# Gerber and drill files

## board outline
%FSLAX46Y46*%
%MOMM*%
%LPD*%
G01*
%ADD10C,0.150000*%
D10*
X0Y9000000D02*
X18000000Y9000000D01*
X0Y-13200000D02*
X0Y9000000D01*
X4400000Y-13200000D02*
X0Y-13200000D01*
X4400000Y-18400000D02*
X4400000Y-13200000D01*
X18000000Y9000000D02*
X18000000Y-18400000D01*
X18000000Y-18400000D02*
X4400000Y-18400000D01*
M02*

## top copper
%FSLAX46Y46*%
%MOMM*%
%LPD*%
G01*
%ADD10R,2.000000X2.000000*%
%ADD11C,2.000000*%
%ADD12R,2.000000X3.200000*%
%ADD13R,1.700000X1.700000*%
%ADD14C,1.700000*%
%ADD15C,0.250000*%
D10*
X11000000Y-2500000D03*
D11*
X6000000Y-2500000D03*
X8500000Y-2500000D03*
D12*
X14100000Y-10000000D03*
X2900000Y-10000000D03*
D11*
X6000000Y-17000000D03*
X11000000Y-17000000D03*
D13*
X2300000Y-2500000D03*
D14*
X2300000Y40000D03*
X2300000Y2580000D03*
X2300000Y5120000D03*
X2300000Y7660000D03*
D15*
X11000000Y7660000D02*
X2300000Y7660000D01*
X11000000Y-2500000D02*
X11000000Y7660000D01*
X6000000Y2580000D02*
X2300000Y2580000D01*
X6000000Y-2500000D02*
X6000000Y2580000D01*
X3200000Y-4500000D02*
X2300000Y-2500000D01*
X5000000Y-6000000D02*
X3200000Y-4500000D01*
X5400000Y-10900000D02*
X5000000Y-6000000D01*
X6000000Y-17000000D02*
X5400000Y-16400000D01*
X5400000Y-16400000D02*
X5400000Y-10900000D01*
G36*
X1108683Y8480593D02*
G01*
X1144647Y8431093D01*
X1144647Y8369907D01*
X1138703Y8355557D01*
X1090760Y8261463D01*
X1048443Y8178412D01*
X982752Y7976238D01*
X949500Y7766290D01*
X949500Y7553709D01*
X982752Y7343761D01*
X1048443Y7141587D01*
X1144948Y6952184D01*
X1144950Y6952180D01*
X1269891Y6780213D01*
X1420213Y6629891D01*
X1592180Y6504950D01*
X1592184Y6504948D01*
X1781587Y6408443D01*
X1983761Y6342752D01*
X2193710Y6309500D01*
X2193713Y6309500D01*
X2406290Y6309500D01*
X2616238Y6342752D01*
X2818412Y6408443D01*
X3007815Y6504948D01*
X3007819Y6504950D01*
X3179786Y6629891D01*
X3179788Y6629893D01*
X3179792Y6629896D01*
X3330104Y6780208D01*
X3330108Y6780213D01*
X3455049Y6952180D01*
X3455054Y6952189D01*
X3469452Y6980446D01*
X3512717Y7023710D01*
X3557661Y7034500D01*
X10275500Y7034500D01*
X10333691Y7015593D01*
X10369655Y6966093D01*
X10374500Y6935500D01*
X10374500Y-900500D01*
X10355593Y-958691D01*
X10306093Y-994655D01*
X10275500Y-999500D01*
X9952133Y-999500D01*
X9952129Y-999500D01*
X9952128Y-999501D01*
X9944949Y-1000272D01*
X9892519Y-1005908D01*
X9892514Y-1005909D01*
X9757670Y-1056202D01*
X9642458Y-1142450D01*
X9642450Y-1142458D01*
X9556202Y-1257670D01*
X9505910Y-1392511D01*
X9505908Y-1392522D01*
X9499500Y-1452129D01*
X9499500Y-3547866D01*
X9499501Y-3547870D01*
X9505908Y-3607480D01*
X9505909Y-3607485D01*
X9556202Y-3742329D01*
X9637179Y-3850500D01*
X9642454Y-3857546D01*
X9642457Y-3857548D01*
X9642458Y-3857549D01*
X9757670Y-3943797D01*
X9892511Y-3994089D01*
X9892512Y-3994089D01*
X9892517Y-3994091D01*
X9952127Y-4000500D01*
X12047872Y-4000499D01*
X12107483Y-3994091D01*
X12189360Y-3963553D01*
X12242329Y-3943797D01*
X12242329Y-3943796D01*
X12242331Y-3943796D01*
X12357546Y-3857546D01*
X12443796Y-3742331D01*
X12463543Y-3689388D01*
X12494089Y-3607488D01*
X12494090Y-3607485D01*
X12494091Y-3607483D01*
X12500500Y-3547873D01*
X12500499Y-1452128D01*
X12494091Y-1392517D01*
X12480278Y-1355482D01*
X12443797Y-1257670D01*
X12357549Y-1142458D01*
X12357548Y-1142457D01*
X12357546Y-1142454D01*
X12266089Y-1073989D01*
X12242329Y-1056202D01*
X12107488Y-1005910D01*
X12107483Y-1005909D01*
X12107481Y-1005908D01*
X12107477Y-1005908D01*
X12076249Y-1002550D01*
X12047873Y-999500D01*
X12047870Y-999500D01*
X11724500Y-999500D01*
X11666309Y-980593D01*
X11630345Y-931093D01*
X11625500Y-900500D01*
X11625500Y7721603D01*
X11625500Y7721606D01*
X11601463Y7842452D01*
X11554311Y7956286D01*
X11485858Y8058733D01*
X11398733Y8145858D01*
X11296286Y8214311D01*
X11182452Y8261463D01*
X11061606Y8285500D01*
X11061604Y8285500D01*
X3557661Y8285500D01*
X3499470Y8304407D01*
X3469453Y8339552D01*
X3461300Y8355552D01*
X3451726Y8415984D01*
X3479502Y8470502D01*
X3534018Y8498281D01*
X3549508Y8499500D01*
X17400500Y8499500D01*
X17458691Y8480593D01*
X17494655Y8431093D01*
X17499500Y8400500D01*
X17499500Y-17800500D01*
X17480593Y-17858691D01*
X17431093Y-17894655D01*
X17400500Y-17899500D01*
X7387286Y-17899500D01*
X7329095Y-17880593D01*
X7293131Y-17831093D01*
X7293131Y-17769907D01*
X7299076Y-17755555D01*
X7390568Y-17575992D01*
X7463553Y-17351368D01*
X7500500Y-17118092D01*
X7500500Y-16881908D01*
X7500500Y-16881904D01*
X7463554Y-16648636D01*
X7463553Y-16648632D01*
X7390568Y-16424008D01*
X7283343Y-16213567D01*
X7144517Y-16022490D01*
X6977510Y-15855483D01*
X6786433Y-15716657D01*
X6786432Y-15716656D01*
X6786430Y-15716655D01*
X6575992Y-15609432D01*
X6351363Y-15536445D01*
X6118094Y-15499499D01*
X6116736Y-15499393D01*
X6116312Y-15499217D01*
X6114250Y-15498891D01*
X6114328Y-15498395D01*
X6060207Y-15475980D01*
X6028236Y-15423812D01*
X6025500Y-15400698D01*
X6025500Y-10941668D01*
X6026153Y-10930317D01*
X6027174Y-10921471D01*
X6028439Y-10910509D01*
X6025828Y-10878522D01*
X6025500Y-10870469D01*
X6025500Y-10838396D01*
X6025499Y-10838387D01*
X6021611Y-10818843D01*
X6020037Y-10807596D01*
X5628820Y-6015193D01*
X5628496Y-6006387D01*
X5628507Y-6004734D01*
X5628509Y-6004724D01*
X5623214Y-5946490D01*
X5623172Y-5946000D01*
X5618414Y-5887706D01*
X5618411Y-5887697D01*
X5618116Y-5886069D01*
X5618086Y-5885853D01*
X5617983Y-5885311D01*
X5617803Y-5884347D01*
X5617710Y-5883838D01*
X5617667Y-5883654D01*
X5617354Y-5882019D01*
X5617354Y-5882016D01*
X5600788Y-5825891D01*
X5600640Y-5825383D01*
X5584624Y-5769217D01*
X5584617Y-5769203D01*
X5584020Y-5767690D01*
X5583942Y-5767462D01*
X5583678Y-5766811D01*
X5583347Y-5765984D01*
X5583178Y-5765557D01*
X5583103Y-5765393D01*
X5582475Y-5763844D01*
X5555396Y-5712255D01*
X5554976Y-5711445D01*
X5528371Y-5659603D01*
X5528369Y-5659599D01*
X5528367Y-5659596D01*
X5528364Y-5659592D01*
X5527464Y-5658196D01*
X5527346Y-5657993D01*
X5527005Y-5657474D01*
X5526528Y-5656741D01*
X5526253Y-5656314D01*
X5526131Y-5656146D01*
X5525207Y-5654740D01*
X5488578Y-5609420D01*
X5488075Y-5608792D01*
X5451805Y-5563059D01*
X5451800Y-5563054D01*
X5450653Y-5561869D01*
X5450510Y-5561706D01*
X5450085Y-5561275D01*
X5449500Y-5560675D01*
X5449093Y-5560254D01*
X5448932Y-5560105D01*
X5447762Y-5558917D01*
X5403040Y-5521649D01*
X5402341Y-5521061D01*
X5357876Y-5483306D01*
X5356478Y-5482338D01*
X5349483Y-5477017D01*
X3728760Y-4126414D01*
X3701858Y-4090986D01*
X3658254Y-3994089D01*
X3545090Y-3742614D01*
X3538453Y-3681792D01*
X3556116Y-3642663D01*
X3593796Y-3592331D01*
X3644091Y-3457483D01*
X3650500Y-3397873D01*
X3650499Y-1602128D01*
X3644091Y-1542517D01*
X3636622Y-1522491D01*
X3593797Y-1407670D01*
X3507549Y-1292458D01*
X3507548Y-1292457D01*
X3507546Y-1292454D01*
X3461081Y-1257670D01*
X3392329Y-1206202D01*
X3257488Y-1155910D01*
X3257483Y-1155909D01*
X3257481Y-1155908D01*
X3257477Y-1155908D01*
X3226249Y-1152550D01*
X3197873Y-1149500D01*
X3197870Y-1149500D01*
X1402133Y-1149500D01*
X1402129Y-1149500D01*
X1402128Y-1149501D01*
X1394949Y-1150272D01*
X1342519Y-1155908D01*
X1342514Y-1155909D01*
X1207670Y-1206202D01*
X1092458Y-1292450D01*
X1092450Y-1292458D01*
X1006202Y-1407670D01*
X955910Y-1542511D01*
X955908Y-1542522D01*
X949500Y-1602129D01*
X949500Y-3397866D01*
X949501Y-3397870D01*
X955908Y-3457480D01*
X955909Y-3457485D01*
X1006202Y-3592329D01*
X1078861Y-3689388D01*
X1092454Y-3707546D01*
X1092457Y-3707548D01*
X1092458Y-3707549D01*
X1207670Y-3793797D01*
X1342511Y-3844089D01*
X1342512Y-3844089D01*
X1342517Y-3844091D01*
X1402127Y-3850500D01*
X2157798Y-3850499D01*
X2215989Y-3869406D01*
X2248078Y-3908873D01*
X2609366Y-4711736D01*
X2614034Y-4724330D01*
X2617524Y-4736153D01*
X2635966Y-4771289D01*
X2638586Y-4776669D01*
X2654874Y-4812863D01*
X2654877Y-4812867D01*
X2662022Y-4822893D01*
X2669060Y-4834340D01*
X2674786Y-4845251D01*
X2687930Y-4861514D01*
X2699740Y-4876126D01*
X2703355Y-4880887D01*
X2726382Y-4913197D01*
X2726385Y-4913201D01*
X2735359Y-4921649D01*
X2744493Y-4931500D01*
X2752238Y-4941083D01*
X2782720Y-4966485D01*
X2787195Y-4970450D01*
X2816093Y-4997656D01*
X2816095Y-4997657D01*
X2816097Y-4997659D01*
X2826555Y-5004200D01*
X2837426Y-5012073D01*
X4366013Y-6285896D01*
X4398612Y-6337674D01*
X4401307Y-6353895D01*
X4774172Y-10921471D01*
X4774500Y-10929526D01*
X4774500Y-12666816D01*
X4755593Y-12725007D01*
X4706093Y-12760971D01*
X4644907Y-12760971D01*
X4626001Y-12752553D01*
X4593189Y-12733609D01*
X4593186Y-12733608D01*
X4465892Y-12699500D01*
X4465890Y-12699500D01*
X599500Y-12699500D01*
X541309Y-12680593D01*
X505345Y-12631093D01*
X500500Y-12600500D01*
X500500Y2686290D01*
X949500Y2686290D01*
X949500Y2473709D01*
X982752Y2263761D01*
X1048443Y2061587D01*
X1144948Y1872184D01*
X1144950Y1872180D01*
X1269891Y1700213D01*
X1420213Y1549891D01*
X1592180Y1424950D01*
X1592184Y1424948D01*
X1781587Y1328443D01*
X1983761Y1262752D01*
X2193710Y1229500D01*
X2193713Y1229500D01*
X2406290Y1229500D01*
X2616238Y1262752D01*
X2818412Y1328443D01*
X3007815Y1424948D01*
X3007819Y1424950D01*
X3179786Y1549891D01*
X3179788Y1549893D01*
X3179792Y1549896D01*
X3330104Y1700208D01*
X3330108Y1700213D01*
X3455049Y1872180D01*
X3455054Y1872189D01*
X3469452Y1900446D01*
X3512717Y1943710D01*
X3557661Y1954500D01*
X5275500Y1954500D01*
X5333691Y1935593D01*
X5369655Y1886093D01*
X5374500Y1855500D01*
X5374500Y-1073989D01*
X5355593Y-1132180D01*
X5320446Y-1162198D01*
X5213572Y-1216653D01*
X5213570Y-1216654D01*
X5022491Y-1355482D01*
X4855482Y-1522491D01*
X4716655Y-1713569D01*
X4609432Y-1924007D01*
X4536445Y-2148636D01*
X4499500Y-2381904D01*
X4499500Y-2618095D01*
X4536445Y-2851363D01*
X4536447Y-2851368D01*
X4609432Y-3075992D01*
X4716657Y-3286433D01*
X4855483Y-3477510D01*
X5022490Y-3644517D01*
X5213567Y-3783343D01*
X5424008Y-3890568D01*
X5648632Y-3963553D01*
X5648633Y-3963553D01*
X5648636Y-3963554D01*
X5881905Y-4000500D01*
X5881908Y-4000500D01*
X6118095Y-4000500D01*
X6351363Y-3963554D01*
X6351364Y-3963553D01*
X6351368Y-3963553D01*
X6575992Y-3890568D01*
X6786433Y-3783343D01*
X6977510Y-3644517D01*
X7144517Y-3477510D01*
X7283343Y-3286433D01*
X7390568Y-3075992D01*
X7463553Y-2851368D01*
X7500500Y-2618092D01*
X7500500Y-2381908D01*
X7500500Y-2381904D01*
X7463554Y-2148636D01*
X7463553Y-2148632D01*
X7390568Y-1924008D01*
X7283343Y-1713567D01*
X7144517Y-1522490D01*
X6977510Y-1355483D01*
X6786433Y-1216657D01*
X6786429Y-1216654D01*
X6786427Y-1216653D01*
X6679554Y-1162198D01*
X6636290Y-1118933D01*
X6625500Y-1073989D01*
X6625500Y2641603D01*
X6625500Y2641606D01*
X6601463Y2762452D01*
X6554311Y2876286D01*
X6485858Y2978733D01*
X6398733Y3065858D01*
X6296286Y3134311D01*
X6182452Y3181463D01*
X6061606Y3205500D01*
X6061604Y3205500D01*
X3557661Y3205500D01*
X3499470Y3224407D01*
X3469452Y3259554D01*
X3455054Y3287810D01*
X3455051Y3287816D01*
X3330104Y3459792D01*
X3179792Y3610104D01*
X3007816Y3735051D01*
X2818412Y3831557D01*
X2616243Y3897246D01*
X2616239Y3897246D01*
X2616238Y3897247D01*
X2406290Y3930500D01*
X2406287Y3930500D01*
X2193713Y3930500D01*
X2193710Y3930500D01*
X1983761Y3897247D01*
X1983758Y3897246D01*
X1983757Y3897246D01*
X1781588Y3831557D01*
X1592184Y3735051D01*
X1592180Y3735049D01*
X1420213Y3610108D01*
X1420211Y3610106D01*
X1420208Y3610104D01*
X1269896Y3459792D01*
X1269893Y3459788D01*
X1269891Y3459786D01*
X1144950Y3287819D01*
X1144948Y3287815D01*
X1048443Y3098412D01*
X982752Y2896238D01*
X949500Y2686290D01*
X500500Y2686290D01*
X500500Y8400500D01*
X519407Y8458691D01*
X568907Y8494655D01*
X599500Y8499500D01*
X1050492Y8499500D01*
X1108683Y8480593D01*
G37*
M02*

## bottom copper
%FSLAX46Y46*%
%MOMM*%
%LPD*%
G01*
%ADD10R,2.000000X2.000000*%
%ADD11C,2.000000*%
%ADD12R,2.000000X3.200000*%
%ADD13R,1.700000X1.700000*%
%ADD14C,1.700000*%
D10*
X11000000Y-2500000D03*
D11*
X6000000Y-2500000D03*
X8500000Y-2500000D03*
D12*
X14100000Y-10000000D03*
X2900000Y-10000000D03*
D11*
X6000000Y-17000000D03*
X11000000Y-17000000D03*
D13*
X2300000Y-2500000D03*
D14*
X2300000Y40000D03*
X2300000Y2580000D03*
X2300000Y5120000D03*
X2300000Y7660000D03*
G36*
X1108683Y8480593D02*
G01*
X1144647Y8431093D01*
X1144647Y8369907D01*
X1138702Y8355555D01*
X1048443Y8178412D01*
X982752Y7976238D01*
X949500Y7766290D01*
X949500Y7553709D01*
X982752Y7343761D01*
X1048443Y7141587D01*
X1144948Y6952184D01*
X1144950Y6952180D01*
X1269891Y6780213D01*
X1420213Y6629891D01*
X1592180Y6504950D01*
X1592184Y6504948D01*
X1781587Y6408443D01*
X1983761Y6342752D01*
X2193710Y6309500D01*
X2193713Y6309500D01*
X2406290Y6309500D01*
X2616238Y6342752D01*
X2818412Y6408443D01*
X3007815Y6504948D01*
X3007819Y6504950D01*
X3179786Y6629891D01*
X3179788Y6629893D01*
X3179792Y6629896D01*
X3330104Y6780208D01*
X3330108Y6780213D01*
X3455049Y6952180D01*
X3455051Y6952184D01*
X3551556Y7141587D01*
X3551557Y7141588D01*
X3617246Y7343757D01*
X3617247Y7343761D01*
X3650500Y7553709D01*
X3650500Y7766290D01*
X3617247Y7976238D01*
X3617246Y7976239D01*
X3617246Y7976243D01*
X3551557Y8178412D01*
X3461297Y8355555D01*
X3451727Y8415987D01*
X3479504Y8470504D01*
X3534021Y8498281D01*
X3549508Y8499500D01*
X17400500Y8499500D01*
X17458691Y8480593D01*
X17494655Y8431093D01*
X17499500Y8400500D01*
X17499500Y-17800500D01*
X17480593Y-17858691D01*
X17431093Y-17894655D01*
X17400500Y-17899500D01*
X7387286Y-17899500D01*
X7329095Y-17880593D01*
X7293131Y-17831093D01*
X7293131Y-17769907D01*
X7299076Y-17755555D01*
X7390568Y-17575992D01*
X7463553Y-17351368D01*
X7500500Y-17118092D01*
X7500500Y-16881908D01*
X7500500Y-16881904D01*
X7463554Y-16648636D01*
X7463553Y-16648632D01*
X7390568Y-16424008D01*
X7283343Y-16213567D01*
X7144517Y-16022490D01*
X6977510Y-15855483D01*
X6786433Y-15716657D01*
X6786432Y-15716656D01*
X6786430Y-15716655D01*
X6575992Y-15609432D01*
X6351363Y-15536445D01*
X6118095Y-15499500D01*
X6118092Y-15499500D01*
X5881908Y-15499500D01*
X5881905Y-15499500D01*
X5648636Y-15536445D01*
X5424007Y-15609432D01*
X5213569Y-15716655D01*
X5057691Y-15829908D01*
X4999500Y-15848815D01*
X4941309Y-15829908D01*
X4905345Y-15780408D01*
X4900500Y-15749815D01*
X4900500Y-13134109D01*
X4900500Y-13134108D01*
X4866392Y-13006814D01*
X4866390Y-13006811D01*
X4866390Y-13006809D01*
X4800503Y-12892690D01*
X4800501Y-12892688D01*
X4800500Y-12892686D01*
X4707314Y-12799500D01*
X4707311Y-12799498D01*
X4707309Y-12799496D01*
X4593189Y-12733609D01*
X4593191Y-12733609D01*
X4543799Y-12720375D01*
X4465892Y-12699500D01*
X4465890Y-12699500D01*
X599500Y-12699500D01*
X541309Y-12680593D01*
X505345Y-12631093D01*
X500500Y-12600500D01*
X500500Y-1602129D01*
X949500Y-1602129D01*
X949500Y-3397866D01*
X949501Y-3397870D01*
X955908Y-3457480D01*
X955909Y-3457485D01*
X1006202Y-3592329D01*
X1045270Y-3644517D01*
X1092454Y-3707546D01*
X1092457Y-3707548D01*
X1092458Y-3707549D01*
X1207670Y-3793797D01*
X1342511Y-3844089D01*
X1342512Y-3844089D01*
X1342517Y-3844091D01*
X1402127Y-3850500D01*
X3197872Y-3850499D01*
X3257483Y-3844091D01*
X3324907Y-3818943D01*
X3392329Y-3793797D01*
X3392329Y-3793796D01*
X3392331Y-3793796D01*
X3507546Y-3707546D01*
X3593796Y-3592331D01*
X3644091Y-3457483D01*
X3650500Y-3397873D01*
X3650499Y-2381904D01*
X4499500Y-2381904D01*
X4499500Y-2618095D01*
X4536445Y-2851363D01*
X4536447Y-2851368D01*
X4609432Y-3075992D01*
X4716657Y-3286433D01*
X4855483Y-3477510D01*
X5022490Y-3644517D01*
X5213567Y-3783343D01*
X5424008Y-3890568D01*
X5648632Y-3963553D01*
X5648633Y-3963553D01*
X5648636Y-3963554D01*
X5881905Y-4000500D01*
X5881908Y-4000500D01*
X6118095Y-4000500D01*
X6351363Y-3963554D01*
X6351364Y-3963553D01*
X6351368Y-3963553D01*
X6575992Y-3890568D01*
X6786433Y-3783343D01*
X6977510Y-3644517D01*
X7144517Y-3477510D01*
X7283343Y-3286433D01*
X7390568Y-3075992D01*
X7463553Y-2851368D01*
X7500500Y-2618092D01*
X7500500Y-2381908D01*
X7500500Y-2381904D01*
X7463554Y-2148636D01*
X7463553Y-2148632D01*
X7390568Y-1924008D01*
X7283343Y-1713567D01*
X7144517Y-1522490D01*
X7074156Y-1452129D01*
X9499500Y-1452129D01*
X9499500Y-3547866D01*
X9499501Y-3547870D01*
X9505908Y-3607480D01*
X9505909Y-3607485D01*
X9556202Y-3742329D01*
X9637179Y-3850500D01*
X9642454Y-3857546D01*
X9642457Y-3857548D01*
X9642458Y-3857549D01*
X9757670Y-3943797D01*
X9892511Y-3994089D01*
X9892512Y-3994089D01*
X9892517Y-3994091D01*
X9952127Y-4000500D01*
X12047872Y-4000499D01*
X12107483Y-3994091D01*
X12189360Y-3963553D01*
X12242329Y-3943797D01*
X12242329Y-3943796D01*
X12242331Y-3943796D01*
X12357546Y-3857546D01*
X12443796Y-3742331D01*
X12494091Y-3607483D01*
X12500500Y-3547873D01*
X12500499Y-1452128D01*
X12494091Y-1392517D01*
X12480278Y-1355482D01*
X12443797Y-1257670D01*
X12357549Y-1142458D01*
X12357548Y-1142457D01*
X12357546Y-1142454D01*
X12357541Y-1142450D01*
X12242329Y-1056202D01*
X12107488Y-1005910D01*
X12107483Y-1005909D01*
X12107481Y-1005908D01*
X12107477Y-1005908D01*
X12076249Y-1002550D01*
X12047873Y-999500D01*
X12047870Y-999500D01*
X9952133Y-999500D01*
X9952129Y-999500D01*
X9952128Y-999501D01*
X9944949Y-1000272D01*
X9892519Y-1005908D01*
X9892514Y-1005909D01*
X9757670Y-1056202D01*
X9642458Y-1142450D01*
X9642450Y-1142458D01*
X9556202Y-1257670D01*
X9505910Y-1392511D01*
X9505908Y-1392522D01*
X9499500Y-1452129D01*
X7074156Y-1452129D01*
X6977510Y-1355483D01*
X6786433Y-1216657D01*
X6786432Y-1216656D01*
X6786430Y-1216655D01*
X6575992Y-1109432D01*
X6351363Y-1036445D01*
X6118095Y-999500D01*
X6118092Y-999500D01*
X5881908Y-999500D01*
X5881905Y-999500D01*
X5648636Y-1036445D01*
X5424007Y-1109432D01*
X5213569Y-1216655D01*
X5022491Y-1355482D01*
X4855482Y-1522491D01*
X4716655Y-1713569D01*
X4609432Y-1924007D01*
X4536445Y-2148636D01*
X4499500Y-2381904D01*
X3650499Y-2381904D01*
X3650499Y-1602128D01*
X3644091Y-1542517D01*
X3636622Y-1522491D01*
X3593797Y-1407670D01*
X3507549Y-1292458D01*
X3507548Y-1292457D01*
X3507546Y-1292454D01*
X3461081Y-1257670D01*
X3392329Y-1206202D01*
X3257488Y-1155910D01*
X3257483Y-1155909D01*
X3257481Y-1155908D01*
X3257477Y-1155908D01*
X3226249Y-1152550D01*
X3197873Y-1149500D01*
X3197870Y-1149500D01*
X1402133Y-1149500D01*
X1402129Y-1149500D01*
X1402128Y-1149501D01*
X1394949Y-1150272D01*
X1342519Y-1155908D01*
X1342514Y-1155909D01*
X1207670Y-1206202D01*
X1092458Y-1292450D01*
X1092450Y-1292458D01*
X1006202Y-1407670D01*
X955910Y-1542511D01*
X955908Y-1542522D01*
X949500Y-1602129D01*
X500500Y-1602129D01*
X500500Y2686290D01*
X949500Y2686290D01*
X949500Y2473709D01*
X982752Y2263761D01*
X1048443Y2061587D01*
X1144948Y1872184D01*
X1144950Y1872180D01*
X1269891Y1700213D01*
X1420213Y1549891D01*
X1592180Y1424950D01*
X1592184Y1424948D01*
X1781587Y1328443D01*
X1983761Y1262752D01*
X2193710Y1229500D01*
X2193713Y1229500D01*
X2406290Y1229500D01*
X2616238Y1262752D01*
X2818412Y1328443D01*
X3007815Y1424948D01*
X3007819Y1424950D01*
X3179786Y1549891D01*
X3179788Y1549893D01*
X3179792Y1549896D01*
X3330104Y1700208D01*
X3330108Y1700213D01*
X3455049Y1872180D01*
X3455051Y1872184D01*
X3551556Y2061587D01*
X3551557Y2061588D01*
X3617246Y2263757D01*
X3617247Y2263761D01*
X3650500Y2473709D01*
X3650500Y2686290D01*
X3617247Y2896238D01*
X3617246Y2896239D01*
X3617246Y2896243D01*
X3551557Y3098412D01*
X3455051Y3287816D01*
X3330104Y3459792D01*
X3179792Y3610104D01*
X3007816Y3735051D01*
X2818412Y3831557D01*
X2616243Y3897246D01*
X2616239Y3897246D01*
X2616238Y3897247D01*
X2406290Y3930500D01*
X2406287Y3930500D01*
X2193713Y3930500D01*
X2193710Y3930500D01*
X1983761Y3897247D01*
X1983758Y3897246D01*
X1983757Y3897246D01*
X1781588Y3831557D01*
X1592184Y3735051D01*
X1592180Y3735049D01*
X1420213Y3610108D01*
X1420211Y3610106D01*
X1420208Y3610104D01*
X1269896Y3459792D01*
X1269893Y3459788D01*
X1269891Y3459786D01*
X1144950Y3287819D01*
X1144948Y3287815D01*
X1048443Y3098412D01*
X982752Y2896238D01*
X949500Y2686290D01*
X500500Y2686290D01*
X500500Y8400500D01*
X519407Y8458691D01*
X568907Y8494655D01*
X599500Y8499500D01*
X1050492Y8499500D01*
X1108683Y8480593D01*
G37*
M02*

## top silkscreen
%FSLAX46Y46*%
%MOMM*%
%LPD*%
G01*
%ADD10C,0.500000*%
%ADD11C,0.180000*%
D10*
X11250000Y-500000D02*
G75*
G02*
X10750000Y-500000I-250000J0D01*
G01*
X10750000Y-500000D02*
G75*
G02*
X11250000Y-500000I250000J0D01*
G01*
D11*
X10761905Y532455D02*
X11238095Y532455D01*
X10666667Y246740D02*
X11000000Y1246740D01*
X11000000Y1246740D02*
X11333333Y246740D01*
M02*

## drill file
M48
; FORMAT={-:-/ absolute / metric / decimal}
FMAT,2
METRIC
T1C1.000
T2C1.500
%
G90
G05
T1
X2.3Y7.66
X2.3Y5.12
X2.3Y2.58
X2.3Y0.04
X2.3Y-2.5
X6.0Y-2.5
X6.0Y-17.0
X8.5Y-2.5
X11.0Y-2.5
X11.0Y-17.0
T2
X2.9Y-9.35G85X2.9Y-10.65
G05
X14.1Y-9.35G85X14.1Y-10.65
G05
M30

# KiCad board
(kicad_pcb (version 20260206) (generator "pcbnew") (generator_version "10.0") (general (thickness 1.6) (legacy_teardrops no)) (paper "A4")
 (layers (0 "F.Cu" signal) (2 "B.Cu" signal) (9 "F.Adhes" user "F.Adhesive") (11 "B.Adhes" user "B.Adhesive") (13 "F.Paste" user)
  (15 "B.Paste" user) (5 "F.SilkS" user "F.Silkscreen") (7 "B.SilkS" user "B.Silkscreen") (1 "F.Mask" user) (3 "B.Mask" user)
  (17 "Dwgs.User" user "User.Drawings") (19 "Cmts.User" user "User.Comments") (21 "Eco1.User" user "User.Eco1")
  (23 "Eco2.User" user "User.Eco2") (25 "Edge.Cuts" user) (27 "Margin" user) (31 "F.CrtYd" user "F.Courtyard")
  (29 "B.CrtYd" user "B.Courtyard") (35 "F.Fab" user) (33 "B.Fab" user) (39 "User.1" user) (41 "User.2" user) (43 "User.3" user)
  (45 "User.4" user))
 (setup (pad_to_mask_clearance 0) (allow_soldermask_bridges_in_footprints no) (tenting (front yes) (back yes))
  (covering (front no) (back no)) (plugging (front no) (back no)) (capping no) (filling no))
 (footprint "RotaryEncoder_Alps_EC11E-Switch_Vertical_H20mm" (layer "F.Cu") (at 11 2.5 -90)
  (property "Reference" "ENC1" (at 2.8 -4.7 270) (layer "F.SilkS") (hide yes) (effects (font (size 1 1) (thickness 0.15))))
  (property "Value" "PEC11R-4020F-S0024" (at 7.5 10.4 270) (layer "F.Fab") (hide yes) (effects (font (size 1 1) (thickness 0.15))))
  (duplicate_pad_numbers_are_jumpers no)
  (pad "A" thru_hole rect (at 0 0 270) (size 2 2) (drill 1) (layers "*.Cu" "*.Mask") (remove_unused_layers no) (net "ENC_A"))
  (pad "B" thru_hole circle (at 0 5 270) (size 2 2) (drill 1) (layers "*.Cu" "*.Mask") (remove_unused_layers no) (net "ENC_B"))
  (pad "C" thru_hole circle (at 0 2.5 270) (size 2 2) (drill 1) (layers "*.Cu" "*.Mask") (remove_unused_layers no) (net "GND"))
  (pad "MP" thru_hole rect (at 7.5 -3.1 270) (size 3.2 2) (drill oval 2.8 1.5) (layers "*.Cu" "*.Mask") (remove_unused_layers no)
   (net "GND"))
  (pad "MP" thru_hole rect (at 7.5 8.1 270) (size 3.2 2) (drill oval 2.8 1.5) (layers "*.Cu" "*.Mask") (remove_unused_layers no) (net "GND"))
  (pad "S1" thru_hole circle (at 14.5 5 270) (size 2 2) (drill 1) (layers "*.Cu" "*.Mask") (remove_unused_layers no) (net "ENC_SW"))
  (pad "S2" thru_hole circle (at 14.5 0 270) (size 2 2) (drill 1) (layers "*.Cu" "*.Mask") (remove_unused_layers no) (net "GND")))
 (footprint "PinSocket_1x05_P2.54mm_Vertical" (layer "B.Cu") (at 2.3 2.5)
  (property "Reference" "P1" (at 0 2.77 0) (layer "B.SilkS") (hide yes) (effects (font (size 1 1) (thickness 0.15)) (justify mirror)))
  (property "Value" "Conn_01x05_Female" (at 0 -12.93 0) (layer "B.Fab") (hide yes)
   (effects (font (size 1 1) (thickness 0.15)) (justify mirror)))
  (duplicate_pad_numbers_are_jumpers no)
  (pad "1" thru_hole rect (at 0 0) (size 1.7 1.7) (drill 1) (layers "*.Cu" "*.Mask") (remove_unused_layers no) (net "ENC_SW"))
  (pad "2" thru_hole circle (at 0 -2.54) (size 1.7 1.7) (drill 1) (layers "*.Cu" "*.Mask") (remove_unused_layers no) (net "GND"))
  (pad "3" thru_hole circle (at 0 -5.08) (size 1.7 1.7) (drill 1) (layers "*.Cu" "*.Mask") (remove_unused_layers no) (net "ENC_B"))
  (pad "4" thru_hole circle (at 0 -7.62) (size 1.7 1.7) (drill 1) (layers "*.Cu" "*.Mask") (remove_unused_layers no) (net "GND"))
  (pad "5" thru_hole circle (at 0 -10.16) (size 1.7 1.7) (drill 1) (layers "*.Cu" "*.Mask") (remove_unused_layers no) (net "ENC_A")))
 (gr_circle (center 11 0.5) (end 11.45 0.5) (stroke (width 0.1) (type default)) (fill yes) (layer "F.SilkS"))
 (gr_line (start 0 -9) (end 18 -9) (stroke (width 0.15) (type default)) (layer "Edge.Cuts"))
 (gr_line (start 0 13.2) (end 0 -9) (stroke (width 0.15) (type default)) (layer "Edge.Cuts"))
 (gr_line (start 4.4 13.2) (end 0 13.2) (stroke (width 0.15) (type default)) (layer "Edge.Cuts"))
 (gr_line (start 4.4 18.4) (end 4.4 13.2) (stroke (width 0.15) (type default)) (layer "Edge.Cuts"))
 (gr_line (start 18 -9) (end 18 18.4) (stroke (width 0.15) (type default)) (layer "Edge.Cuts"))
 (gr_line (start 18 18.4) (end 4.4 18.4) (stroke (width 0.15) (type default)) (layer "Edge.Cuts"))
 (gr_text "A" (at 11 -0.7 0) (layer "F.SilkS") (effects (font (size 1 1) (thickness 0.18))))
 (segment (start 11 -7.66) (end 2.3 -7.66) (width 0.25) (layer "F.Cu") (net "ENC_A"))
 (segment (start 11 2.5) (end 11 -7.66) (width 0.25) (layer "F.Cu") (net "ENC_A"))
 (segment (start 6 -2.58) (end 2.3 -2.58) (width 0.25) (layer "F.Cu") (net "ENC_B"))
 (segment (start 6 2.5) (end 6 -2.58) (width 0.25) (layer "F.Cu") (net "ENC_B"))
 (segment (start 3.2 4.5) (end 2.3 2.5) (width 0.25) (layer "F.Cu") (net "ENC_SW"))
 (segment (start 5 6) (end 3.2 4.5) (width 0.25) (layer "F.Cu") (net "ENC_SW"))
 (segment (start 5.4 10.9) (end 5 6) (width 0.25) (layer "F.Cu") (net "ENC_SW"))
 (segment (start 6 17) (end 5.4 16.4) (width 0.25) (layer "F.Cu") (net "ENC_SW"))
 (segment (start 5.4 16.4) (end 5.4 10.9) (width 0.25) (layer "F.Cu") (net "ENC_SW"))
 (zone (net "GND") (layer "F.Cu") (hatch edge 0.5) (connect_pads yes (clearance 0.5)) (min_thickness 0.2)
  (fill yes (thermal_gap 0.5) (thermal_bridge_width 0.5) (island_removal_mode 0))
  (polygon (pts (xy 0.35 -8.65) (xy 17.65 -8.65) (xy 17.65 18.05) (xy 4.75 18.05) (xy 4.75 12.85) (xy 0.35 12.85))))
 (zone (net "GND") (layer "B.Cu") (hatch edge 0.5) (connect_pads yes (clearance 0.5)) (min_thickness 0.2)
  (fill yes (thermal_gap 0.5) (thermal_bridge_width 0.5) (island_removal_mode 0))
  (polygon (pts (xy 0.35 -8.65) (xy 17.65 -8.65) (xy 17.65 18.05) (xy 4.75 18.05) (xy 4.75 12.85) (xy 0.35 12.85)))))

